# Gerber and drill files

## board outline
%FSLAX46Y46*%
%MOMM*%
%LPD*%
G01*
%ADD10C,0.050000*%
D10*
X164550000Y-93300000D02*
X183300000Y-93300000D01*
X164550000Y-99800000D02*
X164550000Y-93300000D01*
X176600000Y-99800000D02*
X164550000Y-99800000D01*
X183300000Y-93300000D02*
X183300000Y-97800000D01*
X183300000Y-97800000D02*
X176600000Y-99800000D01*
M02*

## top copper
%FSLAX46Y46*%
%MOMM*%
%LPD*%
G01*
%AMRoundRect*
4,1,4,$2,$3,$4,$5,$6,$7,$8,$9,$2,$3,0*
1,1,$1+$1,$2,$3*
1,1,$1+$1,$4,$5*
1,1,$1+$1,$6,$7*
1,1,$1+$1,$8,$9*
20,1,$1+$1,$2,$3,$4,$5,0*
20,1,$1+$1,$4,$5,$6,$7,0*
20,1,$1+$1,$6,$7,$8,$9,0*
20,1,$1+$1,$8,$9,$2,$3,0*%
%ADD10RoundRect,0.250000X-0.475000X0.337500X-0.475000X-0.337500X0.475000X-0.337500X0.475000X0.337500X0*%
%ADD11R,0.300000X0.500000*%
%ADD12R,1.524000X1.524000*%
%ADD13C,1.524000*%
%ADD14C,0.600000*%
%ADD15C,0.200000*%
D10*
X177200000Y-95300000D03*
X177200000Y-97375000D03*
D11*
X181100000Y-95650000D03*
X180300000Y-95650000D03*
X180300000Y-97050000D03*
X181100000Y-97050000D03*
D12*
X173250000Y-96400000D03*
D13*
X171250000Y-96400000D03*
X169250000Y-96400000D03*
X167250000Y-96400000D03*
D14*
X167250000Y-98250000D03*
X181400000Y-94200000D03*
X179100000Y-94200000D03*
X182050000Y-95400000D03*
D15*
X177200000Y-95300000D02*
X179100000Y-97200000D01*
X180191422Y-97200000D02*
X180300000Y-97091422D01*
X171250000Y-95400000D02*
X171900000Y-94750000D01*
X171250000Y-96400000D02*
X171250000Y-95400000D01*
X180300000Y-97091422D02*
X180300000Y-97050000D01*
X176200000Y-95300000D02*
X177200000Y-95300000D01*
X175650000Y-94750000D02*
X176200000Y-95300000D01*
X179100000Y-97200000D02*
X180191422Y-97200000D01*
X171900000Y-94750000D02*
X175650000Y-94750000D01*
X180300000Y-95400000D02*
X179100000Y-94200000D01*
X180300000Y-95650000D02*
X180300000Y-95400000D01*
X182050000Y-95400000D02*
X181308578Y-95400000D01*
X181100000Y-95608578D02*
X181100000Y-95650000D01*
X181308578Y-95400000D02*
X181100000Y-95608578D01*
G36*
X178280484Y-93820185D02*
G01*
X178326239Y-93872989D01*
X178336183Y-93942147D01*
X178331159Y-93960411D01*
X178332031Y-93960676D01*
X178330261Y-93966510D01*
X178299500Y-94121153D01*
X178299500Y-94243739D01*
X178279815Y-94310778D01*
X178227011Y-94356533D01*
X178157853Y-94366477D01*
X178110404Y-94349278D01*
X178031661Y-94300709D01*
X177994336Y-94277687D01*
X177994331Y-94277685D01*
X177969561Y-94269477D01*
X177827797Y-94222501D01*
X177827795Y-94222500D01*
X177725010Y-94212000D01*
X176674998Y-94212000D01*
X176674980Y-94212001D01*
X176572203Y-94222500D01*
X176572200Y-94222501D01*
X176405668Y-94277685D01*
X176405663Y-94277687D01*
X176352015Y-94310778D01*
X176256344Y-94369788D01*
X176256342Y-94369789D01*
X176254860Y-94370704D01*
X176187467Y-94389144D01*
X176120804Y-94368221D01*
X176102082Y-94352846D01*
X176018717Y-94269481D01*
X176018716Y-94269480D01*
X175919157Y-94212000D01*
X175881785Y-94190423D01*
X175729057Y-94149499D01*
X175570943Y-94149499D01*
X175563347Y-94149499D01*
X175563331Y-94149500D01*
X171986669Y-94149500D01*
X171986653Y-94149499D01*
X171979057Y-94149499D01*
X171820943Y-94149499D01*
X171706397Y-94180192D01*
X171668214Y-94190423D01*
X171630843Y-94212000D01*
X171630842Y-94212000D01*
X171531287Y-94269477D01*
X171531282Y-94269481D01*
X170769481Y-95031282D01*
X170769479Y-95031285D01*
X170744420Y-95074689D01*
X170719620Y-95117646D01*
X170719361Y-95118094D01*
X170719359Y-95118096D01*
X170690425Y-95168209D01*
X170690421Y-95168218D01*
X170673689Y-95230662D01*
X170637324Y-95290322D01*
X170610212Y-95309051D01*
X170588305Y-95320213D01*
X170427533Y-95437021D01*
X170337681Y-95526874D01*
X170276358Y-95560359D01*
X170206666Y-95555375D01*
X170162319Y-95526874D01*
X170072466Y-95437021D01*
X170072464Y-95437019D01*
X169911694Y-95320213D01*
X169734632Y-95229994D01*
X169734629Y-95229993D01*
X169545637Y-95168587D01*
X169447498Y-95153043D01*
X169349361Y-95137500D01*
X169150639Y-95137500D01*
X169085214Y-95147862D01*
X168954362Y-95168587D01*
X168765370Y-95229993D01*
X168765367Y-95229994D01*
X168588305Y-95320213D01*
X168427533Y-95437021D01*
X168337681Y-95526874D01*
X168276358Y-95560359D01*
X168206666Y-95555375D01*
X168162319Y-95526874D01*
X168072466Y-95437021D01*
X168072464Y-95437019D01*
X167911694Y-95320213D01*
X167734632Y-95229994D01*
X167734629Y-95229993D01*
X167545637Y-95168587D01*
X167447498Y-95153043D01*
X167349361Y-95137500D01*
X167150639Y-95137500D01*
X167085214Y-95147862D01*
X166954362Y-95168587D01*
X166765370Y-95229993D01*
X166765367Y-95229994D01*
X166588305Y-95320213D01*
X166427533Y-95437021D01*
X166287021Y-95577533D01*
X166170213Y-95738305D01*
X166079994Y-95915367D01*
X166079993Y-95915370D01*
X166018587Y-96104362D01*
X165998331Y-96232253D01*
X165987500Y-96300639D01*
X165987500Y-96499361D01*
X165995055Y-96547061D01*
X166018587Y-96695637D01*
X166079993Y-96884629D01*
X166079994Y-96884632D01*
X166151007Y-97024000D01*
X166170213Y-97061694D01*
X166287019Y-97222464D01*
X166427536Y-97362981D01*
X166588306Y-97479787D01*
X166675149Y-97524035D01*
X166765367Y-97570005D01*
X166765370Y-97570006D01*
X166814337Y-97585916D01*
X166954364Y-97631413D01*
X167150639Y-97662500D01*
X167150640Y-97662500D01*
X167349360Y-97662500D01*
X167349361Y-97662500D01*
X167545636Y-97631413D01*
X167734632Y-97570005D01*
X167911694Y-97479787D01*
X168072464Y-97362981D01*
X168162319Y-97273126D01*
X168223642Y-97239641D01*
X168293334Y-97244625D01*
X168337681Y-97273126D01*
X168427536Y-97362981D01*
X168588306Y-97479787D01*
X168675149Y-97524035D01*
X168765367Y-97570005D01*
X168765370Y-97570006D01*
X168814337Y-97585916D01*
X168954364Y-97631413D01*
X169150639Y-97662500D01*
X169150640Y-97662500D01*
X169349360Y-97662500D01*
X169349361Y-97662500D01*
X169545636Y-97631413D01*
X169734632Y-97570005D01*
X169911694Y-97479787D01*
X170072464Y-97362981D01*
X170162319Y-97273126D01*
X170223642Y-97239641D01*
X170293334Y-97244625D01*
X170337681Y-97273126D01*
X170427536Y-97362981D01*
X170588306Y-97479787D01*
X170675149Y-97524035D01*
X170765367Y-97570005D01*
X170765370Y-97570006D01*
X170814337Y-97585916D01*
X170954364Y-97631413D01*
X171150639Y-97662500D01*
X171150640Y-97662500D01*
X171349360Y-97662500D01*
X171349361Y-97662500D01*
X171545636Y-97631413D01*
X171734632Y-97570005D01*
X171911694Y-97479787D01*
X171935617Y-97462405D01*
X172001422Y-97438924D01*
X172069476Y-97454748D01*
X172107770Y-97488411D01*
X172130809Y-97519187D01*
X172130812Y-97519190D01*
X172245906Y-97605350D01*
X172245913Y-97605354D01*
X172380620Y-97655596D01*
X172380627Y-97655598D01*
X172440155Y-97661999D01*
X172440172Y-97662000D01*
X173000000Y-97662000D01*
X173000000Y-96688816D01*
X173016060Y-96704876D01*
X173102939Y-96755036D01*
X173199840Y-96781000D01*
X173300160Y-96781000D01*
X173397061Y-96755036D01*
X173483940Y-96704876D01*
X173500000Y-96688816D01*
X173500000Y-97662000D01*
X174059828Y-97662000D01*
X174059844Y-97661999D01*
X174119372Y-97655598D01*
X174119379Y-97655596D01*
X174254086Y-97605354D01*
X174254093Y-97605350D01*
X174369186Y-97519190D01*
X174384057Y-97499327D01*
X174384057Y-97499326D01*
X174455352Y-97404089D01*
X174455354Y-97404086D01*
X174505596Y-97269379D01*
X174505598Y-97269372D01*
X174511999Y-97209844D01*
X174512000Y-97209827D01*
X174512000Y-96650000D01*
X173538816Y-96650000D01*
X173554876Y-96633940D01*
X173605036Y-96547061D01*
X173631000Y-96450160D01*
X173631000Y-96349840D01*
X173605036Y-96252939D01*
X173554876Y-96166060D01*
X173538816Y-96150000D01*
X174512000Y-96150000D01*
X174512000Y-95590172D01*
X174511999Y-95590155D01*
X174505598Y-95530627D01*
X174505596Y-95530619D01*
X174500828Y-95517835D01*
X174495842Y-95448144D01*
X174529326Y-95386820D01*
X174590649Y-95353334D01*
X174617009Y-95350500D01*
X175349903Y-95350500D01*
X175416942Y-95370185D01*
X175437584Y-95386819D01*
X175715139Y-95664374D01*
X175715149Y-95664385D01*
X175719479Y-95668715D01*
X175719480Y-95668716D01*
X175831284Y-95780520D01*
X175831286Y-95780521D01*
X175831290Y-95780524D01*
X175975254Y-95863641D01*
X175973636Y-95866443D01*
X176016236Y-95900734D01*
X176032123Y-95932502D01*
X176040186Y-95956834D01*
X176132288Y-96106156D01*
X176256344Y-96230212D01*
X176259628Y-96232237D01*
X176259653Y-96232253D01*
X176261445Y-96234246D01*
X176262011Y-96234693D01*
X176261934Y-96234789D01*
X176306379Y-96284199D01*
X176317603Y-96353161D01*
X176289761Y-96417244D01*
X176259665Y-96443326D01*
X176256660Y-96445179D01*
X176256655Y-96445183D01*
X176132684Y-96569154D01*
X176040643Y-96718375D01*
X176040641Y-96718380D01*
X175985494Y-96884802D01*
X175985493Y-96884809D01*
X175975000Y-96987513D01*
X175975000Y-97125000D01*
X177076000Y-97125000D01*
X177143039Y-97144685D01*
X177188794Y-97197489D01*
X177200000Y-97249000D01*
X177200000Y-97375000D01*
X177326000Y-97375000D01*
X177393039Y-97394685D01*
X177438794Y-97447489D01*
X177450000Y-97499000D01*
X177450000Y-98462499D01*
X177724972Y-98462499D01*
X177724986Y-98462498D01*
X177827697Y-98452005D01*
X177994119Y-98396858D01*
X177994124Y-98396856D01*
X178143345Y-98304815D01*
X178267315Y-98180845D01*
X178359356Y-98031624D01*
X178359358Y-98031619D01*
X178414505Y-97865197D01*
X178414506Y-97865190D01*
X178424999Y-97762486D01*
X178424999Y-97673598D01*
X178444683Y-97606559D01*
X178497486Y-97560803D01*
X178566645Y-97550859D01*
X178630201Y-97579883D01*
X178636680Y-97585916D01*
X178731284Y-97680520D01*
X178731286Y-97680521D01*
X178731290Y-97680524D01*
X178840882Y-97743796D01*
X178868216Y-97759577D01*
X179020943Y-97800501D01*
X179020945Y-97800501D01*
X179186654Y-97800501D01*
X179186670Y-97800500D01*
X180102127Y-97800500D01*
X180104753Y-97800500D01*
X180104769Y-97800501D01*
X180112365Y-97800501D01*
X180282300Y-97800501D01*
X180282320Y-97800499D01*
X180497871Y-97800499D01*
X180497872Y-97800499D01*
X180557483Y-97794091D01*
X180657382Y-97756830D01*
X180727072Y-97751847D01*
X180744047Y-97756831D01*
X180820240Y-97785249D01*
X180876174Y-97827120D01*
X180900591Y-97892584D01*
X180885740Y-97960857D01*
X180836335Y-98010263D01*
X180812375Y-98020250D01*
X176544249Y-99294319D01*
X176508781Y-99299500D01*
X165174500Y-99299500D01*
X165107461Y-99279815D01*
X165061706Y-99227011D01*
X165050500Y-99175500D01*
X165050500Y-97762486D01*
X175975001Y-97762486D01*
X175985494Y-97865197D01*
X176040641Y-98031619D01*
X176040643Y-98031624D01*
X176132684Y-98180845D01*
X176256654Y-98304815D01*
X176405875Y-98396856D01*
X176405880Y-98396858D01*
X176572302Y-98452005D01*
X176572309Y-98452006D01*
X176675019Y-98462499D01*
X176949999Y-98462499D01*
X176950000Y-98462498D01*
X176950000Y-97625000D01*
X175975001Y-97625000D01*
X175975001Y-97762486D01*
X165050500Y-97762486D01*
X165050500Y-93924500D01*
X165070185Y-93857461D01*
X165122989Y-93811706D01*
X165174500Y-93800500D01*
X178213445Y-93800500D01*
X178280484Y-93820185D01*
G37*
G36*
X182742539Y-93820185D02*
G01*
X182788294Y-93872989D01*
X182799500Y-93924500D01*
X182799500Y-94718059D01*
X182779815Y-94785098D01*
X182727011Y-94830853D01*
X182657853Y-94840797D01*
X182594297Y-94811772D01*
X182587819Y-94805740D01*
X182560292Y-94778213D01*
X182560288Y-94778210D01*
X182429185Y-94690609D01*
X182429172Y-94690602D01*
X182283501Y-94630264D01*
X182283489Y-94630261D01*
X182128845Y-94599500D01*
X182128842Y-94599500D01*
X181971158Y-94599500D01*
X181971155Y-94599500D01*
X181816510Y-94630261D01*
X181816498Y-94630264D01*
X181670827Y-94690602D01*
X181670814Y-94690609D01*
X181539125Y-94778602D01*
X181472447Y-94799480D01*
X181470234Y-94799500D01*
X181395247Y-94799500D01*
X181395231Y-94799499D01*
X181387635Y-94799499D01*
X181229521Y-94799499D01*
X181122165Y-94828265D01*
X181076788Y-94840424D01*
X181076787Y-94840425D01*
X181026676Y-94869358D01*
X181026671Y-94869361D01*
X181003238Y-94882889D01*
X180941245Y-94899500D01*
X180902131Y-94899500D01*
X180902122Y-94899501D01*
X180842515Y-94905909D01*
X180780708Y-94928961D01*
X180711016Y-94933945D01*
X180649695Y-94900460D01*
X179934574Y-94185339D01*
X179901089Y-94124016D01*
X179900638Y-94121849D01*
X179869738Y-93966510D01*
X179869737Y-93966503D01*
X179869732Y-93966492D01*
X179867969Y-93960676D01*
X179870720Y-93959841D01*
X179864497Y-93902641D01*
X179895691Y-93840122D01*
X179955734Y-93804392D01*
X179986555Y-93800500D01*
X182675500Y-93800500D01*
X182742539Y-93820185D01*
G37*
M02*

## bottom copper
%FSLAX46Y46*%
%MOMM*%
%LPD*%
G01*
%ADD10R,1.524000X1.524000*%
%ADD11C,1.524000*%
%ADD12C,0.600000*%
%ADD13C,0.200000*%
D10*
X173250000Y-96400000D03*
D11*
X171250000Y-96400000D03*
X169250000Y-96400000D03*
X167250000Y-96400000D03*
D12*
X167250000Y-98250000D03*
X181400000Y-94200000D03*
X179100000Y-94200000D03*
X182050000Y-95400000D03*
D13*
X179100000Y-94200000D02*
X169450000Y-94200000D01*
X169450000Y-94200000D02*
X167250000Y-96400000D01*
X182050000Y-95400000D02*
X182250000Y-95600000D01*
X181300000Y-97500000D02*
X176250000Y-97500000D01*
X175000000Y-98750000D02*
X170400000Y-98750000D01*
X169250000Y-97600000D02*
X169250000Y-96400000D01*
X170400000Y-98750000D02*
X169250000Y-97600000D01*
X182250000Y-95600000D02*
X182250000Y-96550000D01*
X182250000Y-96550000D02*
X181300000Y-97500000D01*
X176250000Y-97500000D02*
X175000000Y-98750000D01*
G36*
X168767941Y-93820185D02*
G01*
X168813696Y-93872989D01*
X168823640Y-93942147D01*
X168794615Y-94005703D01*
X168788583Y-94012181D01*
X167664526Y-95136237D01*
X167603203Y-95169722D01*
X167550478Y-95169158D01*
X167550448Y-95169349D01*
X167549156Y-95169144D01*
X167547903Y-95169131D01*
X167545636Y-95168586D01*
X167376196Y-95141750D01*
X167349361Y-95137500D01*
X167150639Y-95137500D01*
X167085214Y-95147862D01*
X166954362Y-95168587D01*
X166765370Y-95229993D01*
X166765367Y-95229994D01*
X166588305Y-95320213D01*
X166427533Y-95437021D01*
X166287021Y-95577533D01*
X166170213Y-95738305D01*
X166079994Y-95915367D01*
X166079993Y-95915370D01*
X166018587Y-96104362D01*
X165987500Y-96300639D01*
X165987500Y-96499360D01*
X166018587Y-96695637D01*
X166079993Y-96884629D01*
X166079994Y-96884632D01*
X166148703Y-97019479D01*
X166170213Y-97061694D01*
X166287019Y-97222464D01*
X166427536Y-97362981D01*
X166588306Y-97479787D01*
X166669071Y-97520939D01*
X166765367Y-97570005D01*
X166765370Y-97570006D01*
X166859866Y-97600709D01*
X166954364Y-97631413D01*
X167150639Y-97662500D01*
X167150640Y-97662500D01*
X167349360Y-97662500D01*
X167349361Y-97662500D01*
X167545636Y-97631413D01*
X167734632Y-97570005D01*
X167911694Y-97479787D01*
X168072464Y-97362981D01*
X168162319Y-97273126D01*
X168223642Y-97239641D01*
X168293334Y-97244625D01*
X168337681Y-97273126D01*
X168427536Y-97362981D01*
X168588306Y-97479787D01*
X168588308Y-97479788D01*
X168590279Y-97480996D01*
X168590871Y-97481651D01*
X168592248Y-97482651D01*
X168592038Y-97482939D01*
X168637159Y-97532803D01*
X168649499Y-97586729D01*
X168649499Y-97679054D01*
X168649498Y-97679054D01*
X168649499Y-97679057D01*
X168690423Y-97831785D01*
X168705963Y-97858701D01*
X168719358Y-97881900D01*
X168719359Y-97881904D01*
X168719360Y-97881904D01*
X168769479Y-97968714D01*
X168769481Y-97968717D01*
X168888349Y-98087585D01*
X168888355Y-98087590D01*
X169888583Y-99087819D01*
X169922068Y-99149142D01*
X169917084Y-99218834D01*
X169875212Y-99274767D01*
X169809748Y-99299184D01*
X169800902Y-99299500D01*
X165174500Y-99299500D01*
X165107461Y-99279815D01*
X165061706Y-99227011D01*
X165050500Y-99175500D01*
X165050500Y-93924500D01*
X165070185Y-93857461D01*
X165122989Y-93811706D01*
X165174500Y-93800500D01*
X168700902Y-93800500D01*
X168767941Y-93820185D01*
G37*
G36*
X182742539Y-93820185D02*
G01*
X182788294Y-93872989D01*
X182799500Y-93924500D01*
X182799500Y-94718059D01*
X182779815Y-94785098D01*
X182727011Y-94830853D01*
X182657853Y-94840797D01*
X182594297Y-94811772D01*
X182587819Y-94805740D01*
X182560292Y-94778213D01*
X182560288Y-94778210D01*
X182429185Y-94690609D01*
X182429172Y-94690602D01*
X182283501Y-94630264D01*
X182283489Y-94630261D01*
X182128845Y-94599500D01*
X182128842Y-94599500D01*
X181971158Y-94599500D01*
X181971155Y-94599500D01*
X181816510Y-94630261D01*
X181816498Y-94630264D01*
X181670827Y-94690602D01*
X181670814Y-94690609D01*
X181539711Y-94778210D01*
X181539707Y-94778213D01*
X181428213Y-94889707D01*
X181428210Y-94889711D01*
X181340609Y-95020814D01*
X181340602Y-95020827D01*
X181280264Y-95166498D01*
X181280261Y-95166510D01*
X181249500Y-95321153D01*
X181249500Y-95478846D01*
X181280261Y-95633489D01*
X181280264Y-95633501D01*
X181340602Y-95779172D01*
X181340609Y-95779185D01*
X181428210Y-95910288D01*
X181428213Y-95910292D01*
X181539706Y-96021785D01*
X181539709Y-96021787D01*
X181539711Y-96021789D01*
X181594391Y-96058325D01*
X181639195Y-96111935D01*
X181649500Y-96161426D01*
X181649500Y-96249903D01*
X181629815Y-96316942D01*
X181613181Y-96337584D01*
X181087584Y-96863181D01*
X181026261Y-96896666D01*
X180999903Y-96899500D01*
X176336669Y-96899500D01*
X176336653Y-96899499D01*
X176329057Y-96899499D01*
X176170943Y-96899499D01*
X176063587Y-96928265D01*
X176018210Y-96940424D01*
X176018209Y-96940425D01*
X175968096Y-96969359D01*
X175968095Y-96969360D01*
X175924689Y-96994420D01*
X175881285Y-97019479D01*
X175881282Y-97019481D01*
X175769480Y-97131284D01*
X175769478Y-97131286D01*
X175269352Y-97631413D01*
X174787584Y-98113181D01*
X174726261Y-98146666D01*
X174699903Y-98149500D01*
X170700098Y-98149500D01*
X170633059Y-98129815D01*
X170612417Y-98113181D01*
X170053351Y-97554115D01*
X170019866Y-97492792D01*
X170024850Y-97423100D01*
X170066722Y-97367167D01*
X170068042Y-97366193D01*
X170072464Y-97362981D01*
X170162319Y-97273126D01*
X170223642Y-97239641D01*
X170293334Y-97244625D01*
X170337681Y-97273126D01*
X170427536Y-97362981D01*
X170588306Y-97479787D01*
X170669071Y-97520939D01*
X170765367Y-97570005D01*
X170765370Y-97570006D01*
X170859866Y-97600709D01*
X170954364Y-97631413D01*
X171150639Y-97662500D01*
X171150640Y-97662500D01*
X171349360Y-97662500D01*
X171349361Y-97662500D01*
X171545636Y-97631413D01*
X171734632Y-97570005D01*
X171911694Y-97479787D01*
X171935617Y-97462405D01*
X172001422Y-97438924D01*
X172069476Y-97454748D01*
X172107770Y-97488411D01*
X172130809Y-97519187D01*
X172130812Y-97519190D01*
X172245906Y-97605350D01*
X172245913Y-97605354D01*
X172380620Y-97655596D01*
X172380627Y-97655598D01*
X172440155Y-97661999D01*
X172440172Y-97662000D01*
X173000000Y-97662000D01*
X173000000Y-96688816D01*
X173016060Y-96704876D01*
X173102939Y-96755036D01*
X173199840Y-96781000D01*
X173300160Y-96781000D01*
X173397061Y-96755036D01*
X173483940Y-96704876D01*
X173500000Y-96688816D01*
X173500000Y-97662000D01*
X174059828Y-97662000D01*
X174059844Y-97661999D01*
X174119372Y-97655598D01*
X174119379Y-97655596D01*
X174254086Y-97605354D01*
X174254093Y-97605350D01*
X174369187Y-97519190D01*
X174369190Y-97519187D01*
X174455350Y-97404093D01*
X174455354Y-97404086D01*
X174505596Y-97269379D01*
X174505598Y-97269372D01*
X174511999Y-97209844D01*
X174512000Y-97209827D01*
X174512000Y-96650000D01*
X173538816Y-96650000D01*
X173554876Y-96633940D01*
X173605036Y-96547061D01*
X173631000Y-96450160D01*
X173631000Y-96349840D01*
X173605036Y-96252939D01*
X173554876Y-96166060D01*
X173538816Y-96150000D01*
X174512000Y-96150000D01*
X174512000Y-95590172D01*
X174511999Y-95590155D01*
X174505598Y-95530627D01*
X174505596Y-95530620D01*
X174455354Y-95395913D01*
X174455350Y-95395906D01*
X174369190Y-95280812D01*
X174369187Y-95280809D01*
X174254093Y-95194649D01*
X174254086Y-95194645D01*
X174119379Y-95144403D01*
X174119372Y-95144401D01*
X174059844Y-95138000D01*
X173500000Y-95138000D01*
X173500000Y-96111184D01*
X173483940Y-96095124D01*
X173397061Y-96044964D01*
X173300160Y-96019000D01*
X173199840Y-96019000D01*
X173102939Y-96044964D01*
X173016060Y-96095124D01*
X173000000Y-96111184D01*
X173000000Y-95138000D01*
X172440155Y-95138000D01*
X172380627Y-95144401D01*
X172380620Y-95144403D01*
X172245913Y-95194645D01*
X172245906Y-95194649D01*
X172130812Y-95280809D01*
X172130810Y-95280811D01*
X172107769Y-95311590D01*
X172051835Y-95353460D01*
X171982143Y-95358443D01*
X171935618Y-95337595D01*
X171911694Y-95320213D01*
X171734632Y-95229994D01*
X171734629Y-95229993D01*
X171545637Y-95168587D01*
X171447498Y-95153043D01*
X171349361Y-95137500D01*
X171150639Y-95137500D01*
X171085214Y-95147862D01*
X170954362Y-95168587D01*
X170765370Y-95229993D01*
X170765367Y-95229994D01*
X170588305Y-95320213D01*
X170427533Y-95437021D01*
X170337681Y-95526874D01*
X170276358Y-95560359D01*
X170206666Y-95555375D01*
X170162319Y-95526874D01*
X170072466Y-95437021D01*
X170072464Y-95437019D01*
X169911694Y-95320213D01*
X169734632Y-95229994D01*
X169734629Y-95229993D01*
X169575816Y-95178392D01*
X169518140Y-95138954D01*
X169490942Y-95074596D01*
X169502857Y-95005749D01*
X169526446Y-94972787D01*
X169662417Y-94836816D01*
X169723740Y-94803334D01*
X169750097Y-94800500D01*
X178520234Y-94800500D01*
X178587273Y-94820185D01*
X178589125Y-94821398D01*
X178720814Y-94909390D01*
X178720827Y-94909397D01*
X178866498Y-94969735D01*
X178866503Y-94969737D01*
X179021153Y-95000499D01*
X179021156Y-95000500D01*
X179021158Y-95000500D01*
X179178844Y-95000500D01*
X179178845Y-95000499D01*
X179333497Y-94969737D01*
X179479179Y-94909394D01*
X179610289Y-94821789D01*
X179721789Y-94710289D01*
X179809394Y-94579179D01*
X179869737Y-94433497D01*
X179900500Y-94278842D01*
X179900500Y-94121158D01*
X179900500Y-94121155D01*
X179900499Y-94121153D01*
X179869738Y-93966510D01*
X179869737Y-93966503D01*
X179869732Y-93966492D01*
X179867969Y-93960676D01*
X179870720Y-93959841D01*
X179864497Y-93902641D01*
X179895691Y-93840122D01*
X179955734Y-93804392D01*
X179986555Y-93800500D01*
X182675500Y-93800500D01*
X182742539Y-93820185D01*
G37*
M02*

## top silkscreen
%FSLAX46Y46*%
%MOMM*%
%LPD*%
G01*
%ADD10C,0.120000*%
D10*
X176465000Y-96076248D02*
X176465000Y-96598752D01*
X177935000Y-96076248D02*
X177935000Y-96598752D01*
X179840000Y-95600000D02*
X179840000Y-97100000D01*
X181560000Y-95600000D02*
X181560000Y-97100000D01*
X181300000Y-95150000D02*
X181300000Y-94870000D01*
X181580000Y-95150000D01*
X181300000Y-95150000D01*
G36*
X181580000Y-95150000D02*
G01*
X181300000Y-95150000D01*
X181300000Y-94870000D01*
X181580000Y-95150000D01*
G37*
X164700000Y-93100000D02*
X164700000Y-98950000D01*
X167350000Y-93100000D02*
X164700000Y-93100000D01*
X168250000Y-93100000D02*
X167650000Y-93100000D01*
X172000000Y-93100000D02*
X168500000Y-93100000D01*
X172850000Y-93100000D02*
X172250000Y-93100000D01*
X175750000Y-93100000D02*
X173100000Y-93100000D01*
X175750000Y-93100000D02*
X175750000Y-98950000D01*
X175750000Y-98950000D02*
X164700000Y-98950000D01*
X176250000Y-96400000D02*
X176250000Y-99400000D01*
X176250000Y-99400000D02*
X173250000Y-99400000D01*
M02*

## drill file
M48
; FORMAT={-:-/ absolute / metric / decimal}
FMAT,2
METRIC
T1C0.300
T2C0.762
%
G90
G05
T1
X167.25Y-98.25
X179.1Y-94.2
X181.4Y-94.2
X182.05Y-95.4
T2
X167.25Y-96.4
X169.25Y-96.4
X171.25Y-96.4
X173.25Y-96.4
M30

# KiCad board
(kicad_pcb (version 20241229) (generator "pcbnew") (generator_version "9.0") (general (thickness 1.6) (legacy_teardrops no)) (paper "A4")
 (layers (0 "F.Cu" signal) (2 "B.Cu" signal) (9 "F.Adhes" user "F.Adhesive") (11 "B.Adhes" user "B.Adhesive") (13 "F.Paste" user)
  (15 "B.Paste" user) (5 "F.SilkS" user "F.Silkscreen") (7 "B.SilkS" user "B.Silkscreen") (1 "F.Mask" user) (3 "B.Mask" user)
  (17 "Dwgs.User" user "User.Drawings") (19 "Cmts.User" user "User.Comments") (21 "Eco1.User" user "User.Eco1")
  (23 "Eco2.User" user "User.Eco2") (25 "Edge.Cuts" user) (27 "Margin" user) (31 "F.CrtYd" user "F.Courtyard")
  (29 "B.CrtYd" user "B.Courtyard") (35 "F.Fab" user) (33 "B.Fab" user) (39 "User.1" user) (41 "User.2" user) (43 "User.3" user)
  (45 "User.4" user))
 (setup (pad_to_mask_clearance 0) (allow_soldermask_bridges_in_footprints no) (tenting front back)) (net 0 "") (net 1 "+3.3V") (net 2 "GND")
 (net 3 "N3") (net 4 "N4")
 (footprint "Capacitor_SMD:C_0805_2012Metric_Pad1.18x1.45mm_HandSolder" (layer "F.Cu") (at 177.2 96.3375 -90)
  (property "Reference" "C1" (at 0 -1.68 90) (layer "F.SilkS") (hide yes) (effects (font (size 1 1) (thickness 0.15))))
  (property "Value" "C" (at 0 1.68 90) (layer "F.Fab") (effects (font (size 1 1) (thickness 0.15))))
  (fp_line (start -0.261252 0.735) (end 0.261252 0.735) (stroke (width 0.12) (type solid)) (layer "F.SilkS"))
  (fp_line (start -0.261252 -0.735) (end 0.261252 -0.735) (stroke (width 0.12) (type solid)) (layer "F.SilkS"))
  (pad "1" smd roundrect (at -1.0375 0 270) (size 1.175 1.45) (layers "F.Cu" "F.Mask" "F.Paste") (roundrect_rratio 0.212766) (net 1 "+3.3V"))
  (pad "2" smd roundrect (at 1.0375 0 270) (size 1.175 1.45) (layers "F.Cu" "F.Mask" "F.Paste") (roundrect_rratio 0.212766) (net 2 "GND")))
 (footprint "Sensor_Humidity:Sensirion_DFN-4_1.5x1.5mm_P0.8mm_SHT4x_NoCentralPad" (layer "F.Cu") (at 180.7 96.35 -90)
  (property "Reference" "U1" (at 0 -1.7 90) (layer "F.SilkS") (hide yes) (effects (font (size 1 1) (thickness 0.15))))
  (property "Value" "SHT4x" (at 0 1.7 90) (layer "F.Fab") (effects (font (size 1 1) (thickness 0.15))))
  (fp_line (start -0.75 0.86) (end 0.75 0.86) (stroke (width 0.12) (type solid)) (layer "F.SilkS"))
  (fp_line (start -0.75 -0.86) (end 0.75 -0.86) (stroke (width 0.12) (type solid)) (layer "F.SilkS"))
  (fp_poly
   (pts (xy -1.2 -0.6) (xy -1.48 -0.6) (xy -1.2 -0.88) (xy -1.2 -0.6)) (stroke (width 0.12) (type solid)) (fill yes) (layer "F.SilkS"))
  (pad "1" smd rect (at -0.7 -0.4 270) (size 0.5 0.3) (layers "F.Cu" "F.Mask" "F.Paste") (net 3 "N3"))
  (pad "2" smd rect (at -0.7 0.4 270) (size 0.5 0.3) (layers "F.Cu" "F.Mask" "F.Paste") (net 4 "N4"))
  (pad "3" smd rect (at 0.7 0.4 270) (size 0.5 0.3) (layers "F.Cu" "F.Mask" "F.Paste") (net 1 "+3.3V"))
  (pad "4" smd rect (at 0.7 -0.4 270) (size 0.5 0.3) (layers "F.Cu" "F.Mask" "F.Paste") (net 2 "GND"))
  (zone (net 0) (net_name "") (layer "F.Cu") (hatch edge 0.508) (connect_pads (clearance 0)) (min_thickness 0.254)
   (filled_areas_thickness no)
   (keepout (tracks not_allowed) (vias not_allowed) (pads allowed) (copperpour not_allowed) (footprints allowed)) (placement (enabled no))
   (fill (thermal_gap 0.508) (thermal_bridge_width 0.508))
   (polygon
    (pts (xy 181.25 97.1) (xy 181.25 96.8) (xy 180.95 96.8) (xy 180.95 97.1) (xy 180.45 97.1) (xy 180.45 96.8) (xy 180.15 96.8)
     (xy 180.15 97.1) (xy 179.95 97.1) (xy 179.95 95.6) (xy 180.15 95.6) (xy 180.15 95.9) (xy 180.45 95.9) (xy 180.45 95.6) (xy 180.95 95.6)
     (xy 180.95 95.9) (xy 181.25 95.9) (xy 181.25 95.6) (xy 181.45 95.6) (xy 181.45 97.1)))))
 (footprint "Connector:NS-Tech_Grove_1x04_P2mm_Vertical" (layer "F.Cu") (at 173.25 96.4 -90)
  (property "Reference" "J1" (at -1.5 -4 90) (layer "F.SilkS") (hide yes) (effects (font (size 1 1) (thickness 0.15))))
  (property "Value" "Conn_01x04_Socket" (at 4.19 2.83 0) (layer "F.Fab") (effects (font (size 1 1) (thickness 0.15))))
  (fp_line (start -3.3 8.55) (end 2.55 8.55) (stroke (width 0.12) (type solid)) (layer "F.SilkS"))
  (fp_line (start -3.3 5.9) (end -3.3 8.55) (stroke (width 0.12) (type solid)) (layer "F.SilkS"))
  (fp_line (start -3.3 5) (end -3.3 5.6) (stroke (width 0.12) (type solid)) (layer "F.SilkS"))
  (fp_line (start -3.3 1.25) (end -3.3 4.75) (stroke (width 0.12) (type solid)) (layer "F.SilkS"))
  (fp_line (start -3.3 0.4) (end -3.3 1) (stroke (width 0.12) (type solid)) (layer "F.SilkS"))
  (fp_line (start -3.3 -2.5) (end -3.3 0.15) (stroke (width 0.12) (type solid)) (layer "F.SilkS"))
  (fp_line (start -3.3 -2.5) (end 2.55 -2.5) (stroke (width 0.12) (type solid)) (layer "F.SilkS"))
  (fp_line (start 2.55 -2.5) (end 2.55 8.55) (stroke (width 0.12) (type solid)) (layer "F.SilkS"))
  (fp_line (start 0 -3) (end 3 -3) (stroke (width 0.12) (type solid)) (layer "F.SilkS"))
  (fp_line (start 3 -3) (end 3 0) (stroke (width 0.12) (type solid)) (layer "F.SilkS"))
  (pad "1" thru_hole rect (at 0 0 270) (size 1.524 1.524) (drill 0.762) (layers "*.Cu" "*.Mask") (remove_unused_layers no) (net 2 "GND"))
  (pad "2" thru_hole circle (at 0 2 270) (size 1.524 1.524) (drill 0.762) (layers "*.Cu" "*.Mask") (remove_unused_layers no) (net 1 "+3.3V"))
  (pad "3" thru_hole circle (at 0 4 270) (size 1.524 1.524) (drill 0.762) (layers "*.Cu" "*.Mask") (remove_unused_layers no) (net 3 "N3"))
  (pad "4" thru_hole circle (at 0 6 270) (size 1.524 1.524) (drill 0.762) (layers "*.Cu" "*.Mask") (remove_unused_layers no) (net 4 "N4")))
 (gr_line (start 164.55 93.3) (end 183.3 93.3) (stroke (width 0.05) (type default)) (layer "Edge.Cuts"))
 (gr_line (start 164.55 99.8) (end 164.55 93.3) (stroke (width 0.05) (type default)) (layer "Edge.Cuts"))
 (gr_line (start 176.6 99.8) (end 164.55 99.8) (stroke (width 0.05) (type default)) (layer "Edge.Cuts"))
 (gr_line (start 183.3 93.3) (end 183.3 97.8) (stroke (width 0.05) (type default)) (layer "Edge.Cuts"))
 (gr_line (start 183.3 97.8) (end 176.6 99.8) (stroke (width 0.05) (type default)) (layer "Edge.Cuts"))
 (via (at 167.25 98.25) (size 0.6) (drill 0.3) (layers "F.Cu" "B.Cu") (free yes) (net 2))
 (via (at 181.4 94.2) (size 0.6) (drill 0.3) (layers "F.Cu" "B.Cu") (free yes) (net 2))
 (segment (start 177.2 95.3) (end 179.1 97.2) (width 0.2) (layer "F.Cu") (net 1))
 (segment (start 180.191422 97.2) (end 180.3 97.091422) (width 0.2) (layer "F.Cu") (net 1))
 (segment (start 171.25 95.4) (end 171.9 94.75) (width 0.2) (layer "F.Cu") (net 1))
 (segment (start 171.25 96.4) (end 171.25 95.4) (width 0.2) (layer "F.Cu") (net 1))
 (segment (start 180.3 97.091422) (end 180.3 97.05) (width 0.2) (layer "F.Cu") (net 1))
 (segment (start 176.2 95.3) (end 177.2 95.3) (width 0.2) (layer "F.Cu") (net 1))
 (segment (start 175.65 94.75) (end 176.2 95.3) (width 0.2) (layer "F.Cu") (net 1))
 (segment (start 179.1 97.2) (end 180.191422 97.2) (width 0.2) (layer "F.Cu") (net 1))
 (segment (start 171.9 94.75) (end 175.65 94.75) (width 0.2) (layer "F.Cu") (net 1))
 (segment (start 180.3 95.4) (end 179.1 94.2) (width 0.2) (layer "F.Cu") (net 4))
 (segment (start 180.3 95.65) (end 180.3 95.4) (width 0.2) (layer "F.Cu") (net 4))
 (via (at 179.1 94.2) (size 0.6) (drill 0.3) (layers "F.Cu" "B.Cu") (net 4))
 (segment (start 179.1 94.2) (end 169.45 94.2) (width 0.2) (layer "B.Cu") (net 4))
 (segment (start 169.45 94.2) (end 167.25 96.4) (width 0.2) (layer "B.Cu") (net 4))
 (segment (start 182.05 95.4) (end 181.308578 95.4) (width 0.2) (layer "F.Cu") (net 3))
 (segment (start 181.1 95.608578) (end 181.1 95.65) (width 0.2) (layer "F.Cu") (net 3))
 (segment (start 181.308578 95.4) (end 181.1 95.608578) (width 0.2) (layer "F.Cu") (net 3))
 (via (at 182.05 95.4) (size 0.6) (drill 0.3) (layers "F.Cu" "B.Cu") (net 3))
 (segment (start 182.05 95.4) (end 182.25 95.6) (width 0.2) (layer "B.Cu") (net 3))
 (segment (start 181.3 97.5) (end 176.25 97.5) (width 0.2) (layer "B.Cu") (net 3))
 (segment (start 175 98.75) (end 170.4 98.75) (width 0.2) (layer "B.Cu") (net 3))
 (segment (start 169.25 97.6) (end 169.25 96.4) (width 0.2) (layer "B.Cu") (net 3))
 (segment (start 170.4 98.75) (end 169.25 97.6) (width 0.2) (layer "B.Cu") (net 3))
 (segment (start 182.25 95.6) (end 182.25 96.55) (width 0.2) (layer "B.Cu") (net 3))
 (segment (start 182.25 96.55) (end 181.3 97.5) (width 0.2) (layer "B.Cu") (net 3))
 (segment (start 176.25 97.5) (end 175 98.75) (width 0.2) (layer "B.Cu") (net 3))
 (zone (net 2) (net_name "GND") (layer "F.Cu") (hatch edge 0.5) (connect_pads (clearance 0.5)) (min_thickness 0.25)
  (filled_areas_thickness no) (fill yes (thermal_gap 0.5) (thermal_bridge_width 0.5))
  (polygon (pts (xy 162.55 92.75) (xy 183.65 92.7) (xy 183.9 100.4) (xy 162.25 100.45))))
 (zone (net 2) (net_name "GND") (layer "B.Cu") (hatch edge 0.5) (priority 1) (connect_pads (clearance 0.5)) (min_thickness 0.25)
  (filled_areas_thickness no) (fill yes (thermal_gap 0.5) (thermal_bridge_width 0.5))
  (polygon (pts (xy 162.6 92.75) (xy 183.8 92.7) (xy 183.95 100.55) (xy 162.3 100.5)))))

